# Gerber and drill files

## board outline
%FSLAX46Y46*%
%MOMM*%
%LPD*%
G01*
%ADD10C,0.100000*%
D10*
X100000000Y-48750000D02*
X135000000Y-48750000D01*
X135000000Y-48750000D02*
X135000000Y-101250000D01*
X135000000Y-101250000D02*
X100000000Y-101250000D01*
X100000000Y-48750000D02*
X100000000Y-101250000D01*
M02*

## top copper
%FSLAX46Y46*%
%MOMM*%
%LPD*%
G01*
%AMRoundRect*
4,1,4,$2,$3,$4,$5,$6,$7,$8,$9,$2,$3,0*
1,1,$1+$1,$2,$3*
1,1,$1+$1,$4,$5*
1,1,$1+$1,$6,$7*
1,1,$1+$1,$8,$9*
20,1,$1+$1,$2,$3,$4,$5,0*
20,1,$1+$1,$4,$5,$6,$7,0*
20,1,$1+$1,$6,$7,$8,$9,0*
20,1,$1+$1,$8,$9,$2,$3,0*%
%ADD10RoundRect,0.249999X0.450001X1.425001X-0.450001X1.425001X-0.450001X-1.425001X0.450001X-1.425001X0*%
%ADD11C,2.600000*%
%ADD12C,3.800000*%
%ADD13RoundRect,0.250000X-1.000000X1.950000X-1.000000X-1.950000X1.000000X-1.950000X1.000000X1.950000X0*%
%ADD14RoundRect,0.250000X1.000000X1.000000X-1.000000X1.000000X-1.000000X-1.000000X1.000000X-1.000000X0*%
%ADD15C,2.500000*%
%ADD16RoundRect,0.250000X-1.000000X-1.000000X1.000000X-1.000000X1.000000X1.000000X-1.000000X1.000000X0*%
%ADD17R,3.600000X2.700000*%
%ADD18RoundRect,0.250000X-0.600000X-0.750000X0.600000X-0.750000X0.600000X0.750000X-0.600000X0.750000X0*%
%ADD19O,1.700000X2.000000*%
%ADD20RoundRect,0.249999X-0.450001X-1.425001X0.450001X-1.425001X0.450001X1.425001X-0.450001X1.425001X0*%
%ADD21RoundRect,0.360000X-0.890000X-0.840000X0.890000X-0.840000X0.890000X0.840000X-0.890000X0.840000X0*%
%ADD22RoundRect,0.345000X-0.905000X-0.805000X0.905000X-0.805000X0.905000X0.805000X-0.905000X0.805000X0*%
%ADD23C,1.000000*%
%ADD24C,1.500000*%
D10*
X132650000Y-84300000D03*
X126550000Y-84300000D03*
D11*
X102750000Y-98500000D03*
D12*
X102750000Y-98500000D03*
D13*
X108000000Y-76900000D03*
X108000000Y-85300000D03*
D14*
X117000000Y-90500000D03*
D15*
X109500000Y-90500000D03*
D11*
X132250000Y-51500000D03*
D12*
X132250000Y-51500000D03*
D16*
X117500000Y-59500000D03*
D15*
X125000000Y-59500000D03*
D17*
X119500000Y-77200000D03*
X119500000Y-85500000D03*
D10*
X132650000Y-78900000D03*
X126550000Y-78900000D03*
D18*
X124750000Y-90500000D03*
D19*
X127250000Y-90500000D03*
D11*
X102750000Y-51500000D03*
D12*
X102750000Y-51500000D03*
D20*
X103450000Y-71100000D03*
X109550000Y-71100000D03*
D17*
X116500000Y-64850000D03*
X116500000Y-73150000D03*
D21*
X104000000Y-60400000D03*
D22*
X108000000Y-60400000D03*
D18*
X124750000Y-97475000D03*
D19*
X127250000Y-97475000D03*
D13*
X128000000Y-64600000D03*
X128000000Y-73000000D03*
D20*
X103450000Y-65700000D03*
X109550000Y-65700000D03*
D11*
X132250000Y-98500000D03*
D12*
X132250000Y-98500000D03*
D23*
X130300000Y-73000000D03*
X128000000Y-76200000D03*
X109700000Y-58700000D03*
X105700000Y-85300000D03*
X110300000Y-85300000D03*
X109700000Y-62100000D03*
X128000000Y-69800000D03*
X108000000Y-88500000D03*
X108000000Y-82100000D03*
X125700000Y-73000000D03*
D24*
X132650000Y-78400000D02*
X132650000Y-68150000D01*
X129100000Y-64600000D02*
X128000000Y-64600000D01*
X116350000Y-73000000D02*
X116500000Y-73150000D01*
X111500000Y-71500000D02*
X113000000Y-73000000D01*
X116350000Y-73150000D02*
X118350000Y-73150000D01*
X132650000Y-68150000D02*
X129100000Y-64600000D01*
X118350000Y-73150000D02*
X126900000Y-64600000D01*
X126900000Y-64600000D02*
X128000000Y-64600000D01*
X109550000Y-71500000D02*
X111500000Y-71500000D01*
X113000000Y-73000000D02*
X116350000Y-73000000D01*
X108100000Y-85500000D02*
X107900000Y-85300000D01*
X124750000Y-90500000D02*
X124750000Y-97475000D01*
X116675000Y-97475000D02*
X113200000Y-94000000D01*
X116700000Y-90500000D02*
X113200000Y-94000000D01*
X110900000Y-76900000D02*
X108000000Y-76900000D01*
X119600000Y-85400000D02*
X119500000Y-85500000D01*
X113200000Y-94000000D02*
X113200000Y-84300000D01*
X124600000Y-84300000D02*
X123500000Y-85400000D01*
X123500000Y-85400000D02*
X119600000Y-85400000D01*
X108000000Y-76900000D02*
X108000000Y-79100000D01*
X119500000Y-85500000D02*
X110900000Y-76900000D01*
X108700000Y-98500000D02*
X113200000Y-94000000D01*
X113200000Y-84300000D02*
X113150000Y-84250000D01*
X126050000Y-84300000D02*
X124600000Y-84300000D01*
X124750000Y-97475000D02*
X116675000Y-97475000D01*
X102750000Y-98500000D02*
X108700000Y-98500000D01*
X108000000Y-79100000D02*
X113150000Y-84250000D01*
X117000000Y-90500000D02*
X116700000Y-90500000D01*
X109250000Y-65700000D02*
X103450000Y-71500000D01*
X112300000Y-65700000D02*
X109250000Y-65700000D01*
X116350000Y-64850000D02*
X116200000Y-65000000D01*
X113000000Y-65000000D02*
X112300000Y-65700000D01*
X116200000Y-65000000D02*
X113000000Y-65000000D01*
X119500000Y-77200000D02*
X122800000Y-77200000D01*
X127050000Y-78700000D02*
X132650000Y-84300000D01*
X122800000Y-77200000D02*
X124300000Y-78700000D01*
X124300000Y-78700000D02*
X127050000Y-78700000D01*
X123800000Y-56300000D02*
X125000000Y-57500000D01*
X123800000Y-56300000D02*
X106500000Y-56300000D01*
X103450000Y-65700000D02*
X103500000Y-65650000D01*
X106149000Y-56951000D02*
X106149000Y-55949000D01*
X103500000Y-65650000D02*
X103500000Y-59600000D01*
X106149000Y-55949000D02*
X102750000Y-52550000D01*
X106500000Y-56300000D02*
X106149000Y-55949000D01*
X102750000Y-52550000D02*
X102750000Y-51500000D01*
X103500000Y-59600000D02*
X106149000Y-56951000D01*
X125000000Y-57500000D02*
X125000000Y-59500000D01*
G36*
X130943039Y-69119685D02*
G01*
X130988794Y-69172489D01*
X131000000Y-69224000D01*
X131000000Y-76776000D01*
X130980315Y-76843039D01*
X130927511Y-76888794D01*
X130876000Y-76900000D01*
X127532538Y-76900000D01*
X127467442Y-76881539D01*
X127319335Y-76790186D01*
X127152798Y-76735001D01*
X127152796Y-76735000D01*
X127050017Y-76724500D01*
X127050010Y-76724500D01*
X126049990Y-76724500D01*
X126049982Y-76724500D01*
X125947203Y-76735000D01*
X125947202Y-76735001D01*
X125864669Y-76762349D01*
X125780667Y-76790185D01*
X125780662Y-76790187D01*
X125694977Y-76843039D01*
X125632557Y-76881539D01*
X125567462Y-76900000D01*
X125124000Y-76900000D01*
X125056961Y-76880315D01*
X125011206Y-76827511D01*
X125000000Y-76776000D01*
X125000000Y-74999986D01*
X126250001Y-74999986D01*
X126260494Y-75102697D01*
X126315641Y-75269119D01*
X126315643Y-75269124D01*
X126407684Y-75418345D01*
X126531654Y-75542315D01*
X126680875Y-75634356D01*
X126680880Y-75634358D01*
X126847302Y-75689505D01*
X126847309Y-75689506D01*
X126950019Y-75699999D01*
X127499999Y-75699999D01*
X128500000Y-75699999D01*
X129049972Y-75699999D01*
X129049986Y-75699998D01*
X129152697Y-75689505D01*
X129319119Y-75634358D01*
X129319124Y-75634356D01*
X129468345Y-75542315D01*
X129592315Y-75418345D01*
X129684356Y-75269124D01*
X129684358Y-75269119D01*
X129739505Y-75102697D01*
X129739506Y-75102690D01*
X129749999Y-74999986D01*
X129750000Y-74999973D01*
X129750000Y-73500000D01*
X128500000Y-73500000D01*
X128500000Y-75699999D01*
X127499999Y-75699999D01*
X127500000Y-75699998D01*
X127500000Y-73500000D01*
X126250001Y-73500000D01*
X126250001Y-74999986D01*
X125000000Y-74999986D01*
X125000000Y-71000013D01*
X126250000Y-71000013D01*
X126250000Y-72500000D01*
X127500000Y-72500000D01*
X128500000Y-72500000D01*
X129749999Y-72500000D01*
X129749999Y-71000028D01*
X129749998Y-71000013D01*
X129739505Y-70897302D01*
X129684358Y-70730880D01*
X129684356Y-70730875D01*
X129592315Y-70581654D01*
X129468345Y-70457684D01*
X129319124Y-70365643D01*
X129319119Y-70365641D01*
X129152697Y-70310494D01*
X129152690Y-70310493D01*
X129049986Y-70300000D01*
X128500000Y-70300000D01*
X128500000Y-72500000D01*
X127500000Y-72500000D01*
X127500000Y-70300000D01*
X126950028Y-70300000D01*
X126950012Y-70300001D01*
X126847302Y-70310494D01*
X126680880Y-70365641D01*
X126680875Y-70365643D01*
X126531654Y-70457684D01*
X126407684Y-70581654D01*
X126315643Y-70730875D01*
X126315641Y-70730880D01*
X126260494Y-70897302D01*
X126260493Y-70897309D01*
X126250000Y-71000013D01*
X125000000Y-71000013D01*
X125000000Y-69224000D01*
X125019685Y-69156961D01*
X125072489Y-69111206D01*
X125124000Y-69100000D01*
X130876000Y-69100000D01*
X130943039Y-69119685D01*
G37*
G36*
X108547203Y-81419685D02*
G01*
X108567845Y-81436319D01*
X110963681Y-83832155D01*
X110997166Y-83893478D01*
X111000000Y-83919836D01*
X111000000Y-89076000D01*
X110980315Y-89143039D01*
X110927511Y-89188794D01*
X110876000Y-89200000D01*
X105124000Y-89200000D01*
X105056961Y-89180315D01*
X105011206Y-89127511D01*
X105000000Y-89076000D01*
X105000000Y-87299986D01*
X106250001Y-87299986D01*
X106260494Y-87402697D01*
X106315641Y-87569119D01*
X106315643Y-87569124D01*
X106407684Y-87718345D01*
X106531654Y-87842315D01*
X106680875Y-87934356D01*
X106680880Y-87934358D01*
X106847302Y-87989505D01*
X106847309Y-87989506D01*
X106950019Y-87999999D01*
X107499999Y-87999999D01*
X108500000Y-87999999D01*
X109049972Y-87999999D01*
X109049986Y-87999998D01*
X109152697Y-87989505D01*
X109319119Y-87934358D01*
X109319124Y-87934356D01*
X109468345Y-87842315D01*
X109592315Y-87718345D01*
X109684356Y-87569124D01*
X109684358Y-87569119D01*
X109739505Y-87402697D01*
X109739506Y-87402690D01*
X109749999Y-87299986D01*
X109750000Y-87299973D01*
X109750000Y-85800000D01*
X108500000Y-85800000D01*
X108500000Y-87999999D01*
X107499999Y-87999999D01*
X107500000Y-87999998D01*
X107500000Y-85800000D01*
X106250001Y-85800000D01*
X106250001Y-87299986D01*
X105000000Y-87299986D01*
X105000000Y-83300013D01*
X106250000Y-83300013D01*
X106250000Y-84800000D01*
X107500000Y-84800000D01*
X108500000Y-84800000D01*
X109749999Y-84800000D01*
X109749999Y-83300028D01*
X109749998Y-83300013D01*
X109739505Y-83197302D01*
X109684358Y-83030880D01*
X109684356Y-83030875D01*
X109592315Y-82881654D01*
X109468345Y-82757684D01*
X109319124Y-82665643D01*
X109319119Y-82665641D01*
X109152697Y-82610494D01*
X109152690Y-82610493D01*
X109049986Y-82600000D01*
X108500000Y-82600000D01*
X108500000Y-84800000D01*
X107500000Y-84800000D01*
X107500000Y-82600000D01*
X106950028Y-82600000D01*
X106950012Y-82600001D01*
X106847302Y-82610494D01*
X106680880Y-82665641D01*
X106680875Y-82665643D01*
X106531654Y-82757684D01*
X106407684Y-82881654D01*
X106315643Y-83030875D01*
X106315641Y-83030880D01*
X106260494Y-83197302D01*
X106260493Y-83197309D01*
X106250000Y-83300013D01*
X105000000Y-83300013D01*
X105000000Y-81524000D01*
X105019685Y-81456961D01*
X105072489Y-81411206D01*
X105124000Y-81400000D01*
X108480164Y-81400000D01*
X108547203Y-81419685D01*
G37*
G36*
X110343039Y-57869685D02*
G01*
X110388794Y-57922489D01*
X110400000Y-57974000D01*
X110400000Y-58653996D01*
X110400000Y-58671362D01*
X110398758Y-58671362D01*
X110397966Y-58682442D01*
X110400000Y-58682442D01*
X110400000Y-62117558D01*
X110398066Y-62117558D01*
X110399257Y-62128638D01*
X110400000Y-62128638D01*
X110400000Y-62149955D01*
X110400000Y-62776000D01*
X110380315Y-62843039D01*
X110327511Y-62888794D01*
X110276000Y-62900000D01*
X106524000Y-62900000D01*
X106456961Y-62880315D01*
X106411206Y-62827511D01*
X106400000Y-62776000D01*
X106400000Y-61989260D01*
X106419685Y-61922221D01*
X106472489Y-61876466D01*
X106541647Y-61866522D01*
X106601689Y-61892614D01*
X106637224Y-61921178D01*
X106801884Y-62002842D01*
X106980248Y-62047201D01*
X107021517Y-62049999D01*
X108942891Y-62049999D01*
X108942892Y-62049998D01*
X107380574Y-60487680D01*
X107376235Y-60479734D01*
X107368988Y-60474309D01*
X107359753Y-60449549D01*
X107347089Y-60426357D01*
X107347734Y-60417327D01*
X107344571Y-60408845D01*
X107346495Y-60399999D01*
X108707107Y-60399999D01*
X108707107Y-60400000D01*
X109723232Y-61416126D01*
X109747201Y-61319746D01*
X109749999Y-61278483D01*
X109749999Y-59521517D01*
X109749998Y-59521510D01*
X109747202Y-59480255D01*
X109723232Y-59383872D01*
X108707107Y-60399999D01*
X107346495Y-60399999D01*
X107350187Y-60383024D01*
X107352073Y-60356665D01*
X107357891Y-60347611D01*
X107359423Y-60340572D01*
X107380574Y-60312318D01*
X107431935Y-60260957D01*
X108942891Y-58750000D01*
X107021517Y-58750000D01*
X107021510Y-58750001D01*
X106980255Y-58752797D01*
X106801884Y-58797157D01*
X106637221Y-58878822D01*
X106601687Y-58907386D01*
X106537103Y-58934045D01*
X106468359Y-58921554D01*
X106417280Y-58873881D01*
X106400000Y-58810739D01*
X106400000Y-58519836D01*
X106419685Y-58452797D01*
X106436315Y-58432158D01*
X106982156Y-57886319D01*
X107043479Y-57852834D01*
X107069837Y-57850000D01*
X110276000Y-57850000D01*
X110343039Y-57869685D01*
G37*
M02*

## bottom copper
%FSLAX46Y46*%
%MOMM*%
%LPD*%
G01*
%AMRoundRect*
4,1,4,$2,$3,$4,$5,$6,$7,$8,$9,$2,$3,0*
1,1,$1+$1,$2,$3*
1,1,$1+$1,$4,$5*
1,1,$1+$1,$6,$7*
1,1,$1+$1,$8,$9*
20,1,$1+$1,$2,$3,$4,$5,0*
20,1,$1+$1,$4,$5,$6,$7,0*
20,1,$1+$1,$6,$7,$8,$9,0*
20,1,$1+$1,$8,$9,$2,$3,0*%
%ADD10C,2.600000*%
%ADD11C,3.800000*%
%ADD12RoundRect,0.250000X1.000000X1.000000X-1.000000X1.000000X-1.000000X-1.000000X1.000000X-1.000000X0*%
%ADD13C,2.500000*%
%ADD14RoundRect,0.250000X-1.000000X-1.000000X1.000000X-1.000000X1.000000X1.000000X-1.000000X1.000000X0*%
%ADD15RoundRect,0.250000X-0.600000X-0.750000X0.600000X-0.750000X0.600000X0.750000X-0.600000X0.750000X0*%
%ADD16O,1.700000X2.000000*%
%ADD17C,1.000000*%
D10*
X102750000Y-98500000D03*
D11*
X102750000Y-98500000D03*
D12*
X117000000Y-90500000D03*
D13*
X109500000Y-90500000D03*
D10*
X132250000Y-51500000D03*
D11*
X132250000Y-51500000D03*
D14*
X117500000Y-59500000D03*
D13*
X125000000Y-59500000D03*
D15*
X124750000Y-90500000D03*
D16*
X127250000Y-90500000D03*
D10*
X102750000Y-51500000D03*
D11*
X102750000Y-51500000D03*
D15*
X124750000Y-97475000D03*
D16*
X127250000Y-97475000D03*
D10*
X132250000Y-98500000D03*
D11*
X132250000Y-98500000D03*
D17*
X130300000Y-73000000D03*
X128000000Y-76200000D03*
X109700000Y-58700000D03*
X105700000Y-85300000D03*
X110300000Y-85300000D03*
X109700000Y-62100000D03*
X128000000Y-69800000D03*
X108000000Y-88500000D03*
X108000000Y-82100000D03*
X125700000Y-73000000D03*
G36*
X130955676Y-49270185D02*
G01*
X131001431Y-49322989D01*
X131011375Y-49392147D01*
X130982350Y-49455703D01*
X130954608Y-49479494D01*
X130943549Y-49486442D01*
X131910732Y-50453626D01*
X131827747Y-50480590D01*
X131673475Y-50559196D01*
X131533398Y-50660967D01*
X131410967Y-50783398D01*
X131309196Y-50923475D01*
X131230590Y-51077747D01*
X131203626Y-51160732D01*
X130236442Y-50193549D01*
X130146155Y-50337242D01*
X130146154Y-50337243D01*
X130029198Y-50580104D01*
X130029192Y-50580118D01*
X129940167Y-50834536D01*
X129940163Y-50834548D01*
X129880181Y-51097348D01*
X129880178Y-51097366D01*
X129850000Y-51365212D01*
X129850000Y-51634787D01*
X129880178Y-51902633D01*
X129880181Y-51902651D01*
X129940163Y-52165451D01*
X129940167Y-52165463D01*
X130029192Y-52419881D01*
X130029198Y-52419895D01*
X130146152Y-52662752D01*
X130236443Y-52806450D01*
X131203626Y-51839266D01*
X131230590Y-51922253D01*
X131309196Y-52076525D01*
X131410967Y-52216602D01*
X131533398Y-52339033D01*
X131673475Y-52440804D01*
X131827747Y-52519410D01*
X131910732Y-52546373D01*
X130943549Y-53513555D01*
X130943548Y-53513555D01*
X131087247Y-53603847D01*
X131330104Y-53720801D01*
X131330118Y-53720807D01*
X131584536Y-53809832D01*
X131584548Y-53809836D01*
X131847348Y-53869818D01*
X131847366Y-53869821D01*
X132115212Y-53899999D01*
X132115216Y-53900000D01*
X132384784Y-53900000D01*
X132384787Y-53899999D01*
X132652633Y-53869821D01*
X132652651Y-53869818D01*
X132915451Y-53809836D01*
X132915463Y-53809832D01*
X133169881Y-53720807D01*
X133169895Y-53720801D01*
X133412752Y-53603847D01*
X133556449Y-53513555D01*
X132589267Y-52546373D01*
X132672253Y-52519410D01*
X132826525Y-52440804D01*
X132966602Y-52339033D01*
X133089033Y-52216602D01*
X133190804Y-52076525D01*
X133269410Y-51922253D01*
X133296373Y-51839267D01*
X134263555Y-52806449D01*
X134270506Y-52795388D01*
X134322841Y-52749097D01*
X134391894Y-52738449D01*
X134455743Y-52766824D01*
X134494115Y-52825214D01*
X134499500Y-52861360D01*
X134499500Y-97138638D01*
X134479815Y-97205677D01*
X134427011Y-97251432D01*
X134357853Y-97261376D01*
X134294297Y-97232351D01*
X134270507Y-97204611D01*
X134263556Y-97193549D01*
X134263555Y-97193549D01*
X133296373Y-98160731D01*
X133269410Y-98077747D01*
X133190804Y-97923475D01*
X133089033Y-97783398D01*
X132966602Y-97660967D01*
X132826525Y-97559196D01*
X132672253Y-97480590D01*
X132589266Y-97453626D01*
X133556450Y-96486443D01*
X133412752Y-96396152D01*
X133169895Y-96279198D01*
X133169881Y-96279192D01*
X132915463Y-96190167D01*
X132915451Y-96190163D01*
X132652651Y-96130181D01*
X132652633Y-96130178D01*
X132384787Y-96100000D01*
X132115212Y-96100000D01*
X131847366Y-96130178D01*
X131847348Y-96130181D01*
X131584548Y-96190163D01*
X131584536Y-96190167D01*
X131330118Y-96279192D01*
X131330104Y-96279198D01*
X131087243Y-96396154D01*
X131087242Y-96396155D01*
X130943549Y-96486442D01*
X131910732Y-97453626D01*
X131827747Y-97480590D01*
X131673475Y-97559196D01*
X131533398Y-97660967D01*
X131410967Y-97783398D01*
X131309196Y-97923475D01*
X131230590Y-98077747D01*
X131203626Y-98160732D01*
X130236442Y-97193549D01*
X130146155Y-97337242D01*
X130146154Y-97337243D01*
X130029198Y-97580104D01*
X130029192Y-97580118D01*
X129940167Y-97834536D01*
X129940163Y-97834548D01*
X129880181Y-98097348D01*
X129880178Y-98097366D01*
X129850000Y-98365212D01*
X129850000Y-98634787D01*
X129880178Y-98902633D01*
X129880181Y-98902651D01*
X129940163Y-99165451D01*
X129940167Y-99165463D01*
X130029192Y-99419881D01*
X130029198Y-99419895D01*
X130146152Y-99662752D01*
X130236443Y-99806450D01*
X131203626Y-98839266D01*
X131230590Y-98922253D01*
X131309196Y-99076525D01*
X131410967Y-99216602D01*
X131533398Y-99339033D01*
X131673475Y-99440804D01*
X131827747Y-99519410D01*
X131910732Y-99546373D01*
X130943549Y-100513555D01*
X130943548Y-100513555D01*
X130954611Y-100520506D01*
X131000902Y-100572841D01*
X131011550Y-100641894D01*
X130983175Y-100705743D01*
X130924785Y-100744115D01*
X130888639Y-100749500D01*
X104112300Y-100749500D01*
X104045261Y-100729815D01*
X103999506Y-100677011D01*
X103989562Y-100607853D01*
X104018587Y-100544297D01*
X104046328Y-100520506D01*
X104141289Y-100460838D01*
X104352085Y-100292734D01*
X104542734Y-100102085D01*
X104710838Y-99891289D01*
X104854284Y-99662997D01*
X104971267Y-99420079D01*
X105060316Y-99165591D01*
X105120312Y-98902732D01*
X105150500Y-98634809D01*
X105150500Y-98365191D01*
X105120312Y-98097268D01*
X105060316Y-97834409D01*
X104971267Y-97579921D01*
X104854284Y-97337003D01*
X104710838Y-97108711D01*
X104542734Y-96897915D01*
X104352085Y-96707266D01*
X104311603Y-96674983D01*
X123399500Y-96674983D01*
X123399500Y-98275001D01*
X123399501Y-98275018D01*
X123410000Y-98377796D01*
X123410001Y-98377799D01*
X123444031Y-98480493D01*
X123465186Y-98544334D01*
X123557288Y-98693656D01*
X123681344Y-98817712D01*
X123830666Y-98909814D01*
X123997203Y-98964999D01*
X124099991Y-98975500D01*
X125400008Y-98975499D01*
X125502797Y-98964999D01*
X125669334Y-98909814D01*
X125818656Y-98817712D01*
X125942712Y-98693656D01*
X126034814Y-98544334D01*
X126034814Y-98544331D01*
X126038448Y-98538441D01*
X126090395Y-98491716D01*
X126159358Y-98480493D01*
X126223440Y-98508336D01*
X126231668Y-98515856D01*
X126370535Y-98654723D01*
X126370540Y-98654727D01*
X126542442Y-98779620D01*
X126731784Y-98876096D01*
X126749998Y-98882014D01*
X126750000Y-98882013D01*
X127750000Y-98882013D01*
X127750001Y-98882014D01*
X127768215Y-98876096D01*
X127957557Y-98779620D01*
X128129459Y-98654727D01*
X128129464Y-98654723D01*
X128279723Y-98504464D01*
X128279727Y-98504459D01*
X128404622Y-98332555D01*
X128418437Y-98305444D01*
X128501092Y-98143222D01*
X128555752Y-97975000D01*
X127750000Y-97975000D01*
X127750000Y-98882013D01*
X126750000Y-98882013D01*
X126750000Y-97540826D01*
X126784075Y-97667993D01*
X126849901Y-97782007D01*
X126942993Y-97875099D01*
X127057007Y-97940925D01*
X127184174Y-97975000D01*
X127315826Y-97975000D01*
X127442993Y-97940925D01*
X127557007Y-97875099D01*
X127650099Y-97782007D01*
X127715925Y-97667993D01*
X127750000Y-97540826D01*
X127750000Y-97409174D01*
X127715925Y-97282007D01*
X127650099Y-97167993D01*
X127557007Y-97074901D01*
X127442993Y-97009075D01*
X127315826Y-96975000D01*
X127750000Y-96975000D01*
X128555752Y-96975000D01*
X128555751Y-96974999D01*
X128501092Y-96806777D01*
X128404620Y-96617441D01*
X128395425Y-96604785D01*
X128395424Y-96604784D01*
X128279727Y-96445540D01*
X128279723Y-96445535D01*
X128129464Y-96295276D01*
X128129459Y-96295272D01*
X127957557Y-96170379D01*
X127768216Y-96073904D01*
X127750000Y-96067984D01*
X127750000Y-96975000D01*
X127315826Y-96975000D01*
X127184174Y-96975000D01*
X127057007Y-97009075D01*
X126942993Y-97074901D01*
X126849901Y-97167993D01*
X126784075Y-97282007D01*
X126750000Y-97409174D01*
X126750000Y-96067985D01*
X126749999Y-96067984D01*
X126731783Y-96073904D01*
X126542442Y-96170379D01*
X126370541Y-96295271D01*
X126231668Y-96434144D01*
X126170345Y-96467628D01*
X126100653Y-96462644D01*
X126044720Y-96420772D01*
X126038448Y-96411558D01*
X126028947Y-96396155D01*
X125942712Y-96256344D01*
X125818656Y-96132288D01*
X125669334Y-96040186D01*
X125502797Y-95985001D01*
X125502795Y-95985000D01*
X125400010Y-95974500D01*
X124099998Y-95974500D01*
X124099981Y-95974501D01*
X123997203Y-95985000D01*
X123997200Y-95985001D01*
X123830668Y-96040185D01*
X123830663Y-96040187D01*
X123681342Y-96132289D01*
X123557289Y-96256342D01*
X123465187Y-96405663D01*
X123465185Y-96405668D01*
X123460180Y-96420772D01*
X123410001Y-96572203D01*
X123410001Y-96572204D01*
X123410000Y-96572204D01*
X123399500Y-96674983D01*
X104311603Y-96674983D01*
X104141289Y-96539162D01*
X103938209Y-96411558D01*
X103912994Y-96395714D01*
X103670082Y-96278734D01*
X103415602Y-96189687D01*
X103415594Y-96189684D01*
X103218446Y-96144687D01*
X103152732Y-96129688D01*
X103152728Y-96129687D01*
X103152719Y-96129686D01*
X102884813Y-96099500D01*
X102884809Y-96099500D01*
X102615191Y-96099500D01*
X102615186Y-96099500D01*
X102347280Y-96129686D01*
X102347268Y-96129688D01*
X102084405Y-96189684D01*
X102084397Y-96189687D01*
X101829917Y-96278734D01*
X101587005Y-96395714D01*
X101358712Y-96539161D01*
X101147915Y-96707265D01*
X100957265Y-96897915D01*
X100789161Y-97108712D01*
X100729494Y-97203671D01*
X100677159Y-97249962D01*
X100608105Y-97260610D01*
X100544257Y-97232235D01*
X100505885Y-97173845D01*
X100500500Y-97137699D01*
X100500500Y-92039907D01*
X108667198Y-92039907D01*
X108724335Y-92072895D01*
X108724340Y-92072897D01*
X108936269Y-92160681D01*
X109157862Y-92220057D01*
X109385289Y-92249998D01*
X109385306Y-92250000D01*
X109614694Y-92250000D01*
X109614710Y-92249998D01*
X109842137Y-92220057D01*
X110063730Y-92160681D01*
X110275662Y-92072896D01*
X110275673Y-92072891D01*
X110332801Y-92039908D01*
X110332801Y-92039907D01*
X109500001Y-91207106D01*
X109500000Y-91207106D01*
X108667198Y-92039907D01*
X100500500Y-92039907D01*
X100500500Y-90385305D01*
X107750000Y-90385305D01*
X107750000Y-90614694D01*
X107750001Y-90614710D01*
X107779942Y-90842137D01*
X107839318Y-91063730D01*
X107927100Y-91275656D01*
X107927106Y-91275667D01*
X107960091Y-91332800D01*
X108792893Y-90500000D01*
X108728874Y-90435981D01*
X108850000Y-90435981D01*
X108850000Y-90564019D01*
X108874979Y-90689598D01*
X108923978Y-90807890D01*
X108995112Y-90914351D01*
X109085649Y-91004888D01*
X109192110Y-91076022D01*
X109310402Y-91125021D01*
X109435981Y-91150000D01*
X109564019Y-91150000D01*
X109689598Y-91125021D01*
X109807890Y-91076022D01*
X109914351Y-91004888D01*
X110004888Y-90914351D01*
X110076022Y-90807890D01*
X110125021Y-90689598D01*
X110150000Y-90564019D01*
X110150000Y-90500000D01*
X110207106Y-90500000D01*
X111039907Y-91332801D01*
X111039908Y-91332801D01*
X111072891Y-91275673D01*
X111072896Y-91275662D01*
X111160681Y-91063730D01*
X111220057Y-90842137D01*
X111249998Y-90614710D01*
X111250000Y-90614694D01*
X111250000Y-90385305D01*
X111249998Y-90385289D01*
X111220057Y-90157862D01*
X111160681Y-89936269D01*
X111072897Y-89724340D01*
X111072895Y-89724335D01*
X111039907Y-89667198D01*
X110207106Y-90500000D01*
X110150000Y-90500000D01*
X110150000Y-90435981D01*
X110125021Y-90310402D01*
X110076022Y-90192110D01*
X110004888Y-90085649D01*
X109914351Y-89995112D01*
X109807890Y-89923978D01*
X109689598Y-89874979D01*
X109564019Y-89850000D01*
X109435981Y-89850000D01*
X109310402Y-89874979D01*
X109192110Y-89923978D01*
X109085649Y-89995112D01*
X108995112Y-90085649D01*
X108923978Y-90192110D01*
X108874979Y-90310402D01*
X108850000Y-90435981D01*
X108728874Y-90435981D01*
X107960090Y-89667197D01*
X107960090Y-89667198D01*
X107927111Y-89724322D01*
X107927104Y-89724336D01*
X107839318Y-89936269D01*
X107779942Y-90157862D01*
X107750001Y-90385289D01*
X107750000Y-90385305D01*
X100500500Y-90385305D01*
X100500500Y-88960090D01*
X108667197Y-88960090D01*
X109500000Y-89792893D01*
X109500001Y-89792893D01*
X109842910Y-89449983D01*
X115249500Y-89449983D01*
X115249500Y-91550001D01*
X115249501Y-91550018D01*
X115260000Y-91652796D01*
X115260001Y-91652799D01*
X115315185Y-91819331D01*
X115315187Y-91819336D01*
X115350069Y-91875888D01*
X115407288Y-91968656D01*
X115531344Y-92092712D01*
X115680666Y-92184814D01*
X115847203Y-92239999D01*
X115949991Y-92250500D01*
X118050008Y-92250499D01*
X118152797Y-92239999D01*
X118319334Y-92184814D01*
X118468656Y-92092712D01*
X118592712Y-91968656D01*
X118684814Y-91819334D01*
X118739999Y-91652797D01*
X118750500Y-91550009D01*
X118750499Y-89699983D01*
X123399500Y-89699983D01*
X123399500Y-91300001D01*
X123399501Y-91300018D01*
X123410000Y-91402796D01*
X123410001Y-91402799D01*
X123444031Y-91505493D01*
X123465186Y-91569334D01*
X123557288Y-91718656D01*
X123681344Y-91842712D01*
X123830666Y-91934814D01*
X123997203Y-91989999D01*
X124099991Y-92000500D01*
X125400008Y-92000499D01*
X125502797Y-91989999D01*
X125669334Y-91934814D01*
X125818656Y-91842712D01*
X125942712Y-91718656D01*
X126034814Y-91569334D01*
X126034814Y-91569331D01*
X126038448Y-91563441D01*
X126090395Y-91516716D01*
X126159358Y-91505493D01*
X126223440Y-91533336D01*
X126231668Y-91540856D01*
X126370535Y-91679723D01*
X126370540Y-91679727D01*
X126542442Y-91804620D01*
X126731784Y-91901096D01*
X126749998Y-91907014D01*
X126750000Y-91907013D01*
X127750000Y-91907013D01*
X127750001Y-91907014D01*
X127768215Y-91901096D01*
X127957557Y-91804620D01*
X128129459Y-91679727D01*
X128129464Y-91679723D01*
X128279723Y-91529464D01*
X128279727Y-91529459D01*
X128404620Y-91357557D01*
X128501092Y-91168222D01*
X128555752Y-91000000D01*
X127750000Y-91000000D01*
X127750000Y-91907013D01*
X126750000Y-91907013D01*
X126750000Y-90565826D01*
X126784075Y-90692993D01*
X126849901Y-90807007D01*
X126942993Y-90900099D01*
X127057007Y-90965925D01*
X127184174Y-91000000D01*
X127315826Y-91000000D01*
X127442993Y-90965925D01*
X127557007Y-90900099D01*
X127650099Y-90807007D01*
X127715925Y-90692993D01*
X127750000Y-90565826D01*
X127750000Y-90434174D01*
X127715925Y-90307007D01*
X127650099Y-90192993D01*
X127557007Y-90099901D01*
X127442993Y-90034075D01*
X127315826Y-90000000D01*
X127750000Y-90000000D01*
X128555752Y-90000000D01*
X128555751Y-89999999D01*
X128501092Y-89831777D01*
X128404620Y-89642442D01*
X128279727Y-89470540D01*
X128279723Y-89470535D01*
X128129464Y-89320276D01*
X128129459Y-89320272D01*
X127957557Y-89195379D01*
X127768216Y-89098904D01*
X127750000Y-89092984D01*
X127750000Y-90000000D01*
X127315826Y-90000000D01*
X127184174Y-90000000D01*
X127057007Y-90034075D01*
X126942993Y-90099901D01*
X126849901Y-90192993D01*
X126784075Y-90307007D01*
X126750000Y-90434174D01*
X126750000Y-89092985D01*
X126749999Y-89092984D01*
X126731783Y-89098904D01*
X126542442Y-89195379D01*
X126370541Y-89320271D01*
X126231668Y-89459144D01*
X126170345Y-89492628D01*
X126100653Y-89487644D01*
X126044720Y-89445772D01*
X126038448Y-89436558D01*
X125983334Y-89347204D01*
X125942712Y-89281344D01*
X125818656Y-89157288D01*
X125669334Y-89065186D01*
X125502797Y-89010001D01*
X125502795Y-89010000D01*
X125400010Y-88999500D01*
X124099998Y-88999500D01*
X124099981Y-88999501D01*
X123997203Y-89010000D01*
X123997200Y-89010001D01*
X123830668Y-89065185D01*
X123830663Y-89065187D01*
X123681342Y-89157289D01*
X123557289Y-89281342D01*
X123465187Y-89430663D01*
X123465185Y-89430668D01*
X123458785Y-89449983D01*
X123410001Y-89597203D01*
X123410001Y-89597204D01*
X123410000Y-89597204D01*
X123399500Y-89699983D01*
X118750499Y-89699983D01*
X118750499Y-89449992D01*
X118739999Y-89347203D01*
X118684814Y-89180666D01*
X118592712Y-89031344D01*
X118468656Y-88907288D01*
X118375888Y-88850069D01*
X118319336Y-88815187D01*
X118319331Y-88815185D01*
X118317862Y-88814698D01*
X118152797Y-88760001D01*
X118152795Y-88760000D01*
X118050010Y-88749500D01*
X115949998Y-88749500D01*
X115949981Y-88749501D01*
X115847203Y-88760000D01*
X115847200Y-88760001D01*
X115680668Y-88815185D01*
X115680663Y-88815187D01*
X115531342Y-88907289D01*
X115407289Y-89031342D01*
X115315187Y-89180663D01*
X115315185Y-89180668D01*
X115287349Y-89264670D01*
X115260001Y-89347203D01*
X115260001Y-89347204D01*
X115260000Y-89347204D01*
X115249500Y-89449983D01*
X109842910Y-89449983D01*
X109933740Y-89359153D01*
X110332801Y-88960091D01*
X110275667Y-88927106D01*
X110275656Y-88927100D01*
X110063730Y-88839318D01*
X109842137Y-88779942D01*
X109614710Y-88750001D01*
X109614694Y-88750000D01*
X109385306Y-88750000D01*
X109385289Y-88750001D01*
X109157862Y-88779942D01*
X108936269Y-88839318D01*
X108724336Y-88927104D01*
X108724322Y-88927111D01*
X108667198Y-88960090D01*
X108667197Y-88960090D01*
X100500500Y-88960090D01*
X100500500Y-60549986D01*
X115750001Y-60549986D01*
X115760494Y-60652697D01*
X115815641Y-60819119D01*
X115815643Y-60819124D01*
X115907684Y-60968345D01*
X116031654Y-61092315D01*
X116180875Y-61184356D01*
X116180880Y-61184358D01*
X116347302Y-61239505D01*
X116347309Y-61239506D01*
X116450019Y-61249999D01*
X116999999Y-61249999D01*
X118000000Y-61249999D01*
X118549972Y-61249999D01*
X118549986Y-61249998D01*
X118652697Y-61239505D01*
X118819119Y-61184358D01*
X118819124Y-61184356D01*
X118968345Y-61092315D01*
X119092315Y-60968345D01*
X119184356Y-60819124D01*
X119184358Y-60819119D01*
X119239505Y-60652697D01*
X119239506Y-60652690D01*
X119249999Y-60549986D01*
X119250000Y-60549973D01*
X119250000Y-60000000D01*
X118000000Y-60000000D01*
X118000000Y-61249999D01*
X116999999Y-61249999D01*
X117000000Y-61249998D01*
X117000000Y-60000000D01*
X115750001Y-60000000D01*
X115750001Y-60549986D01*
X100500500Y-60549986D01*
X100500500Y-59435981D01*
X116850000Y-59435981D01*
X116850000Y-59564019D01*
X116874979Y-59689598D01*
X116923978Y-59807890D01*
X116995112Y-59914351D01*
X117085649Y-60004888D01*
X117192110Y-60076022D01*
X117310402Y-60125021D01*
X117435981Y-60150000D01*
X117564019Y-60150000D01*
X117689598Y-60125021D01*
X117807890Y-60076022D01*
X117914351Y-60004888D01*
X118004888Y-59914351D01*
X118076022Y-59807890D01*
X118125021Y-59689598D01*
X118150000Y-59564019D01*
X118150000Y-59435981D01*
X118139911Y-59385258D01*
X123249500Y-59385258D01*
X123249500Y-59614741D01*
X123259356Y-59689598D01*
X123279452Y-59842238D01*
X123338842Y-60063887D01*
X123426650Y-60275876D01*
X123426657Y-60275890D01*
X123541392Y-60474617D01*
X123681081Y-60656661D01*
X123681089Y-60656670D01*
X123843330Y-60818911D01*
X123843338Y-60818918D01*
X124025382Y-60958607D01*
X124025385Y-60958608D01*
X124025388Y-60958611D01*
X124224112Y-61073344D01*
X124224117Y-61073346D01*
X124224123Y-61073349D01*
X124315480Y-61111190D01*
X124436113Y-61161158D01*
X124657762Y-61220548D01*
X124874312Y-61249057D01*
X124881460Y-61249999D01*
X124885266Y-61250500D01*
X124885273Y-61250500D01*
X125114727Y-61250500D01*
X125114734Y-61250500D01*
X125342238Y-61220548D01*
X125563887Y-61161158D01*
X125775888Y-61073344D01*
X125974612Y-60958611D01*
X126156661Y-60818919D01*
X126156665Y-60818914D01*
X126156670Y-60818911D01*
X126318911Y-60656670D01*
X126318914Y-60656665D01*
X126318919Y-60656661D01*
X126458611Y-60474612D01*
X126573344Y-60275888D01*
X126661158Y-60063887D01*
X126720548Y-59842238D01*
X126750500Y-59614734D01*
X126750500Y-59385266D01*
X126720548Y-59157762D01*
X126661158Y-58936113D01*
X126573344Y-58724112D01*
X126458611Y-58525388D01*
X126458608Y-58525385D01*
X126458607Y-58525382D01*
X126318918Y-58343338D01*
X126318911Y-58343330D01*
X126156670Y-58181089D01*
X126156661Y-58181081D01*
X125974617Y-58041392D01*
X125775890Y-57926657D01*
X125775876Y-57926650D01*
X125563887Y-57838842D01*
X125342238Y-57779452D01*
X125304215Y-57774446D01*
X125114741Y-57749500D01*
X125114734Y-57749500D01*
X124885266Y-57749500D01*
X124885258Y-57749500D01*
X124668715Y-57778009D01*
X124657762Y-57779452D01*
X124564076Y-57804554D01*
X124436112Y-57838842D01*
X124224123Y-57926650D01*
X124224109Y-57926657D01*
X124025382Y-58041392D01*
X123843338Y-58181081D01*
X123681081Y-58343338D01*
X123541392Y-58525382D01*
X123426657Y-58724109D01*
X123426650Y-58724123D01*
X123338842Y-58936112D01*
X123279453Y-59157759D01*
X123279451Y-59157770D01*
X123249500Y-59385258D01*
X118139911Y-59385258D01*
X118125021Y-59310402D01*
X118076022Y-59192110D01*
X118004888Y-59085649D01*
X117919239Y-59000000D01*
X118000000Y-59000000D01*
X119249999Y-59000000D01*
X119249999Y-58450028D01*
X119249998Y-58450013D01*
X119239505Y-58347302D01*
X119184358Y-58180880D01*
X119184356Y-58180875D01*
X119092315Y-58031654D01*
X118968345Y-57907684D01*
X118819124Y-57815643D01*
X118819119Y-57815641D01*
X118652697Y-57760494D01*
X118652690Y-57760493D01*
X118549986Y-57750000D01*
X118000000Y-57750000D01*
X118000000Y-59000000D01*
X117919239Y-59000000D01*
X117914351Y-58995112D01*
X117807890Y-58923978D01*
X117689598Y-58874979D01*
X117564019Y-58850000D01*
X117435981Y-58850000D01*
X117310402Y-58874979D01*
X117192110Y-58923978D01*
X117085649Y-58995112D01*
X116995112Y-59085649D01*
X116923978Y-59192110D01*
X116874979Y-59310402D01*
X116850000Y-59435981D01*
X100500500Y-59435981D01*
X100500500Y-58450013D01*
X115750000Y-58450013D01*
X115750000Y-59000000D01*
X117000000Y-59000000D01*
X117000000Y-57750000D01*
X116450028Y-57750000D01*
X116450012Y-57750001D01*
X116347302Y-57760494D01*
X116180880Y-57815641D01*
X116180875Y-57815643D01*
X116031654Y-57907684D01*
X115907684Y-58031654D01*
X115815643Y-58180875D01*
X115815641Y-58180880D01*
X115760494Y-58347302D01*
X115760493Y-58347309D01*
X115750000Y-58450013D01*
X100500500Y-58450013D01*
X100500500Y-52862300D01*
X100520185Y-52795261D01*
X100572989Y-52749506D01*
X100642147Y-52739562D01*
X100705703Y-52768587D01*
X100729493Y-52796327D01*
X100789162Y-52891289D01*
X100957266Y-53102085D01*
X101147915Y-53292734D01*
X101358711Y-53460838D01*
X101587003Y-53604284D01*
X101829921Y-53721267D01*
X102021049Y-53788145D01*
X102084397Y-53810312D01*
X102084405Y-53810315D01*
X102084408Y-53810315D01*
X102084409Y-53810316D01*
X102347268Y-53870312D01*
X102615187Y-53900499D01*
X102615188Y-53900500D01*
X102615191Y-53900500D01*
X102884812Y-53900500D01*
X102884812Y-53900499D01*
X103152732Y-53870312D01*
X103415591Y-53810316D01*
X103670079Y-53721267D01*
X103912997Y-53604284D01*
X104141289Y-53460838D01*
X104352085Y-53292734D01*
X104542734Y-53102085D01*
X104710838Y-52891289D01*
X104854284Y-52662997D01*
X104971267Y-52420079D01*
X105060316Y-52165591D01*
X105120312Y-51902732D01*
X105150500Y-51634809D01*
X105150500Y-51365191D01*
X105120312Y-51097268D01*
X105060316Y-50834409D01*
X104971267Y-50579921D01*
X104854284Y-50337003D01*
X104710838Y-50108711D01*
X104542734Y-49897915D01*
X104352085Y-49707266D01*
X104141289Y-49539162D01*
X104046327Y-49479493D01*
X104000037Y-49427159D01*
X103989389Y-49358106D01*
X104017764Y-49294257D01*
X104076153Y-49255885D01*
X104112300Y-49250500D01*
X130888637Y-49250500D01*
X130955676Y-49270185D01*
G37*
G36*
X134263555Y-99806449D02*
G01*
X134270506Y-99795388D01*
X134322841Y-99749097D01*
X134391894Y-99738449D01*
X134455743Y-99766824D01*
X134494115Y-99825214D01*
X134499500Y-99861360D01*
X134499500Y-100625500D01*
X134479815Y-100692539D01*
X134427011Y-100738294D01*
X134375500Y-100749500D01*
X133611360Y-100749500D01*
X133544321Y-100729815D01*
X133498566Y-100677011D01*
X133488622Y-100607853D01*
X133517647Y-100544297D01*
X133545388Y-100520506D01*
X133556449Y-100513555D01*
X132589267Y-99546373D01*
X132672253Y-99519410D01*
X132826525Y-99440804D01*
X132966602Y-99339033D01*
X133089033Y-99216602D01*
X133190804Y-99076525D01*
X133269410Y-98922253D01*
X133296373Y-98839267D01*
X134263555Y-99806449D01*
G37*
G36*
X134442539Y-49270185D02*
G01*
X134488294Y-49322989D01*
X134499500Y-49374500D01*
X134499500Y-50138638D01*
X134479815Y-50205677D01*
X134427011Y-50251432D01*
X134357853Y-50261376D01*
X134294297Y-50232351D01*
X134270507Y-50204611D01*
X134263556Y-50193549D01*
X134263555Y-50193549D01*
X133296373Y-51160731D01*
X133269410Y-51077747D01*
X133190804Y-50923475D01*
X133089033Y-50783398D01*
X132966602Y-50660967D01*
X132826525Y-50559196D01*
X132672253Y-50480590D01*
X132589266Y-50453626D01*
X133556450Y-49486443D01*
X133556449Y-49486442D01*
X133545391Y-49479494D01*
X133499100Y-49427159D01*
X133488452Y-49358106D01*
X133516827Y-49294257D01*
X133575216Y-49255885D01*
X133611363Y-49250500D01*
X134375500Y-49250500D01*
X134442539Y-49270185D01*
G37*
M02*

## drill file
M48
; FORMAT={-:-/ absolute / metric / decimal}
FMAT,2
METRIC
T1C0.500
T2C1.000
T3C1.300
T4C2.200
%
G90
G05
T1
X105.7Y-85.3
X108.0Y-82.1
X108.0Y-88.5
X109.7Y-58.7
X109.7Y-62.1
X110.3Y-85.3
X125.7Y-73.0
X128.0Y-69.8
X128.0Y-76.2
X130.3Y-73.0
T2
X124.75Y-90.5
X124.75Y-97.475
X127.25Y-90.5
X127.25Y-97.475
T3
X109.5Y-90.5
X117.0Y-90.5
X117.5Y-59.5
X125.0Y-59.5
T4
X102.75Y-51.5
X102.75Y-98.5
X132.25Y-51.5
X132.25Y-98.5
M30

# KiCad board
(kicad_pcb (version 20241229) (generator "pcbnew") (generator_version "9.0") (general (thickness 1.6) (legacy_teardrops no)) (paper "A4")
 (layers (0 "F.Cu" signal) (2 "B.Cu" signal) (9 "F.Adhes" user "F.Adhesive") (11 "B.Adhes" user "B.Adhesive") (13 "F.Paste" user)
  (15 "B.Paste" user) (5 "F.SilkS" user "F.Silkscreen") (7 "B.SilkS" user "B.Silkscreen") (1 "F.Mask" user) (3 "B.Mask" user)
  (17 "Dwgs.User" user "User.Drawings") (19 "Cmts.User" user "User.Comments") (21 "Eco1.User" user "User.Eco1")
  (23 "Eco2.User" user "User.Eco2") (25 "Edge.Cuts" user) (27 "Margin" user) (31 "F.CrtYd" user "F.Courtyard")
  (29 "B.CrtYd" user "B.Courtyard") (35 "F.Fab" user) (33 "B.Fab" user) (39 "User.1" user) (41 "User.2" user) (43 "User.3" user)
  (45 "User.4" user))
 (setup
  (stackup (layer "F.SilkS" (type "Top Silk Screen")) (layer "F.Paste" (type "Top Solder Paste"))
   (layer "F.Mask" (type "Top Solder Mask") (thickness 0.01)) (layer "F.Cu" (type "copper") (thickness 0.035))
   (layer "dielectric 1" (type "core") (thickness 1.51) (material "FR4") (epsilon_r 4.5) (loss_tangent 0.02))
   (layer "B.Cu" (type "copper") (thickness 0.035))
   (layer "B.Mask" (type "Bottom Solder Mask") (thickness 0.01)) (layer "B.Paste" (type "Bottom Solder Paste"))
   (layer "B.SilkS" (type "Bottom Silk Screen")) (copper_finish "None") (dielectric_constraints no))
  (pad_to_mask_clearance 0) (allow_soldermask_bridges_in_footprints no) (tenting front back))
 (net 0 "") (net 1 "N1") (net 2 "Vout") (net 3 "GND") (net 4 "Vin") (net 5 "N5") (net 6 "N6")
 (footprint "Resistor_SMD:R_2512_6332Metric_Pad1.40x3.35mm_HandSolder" (layer "F.Cu") (at 129.6 84.3 180)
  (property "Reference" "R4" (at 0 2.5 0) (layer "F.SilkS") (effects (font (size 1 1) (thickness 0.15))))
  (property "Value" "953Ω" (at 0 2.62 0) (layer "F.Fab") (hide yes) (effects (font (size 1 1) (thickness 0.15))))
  (pad "1" smd roundrect (at -3.05 0 180) (size 1.4 3.35) (layers "F.Cu" "F.Mask" "F.Paste") (roundrect_rratio 0.178571) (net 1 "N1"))
  (pad "2" smd roundrect (at 3.05 0 180) (size 1.4 3.35) (layers "F.Cu" "F.Mask" "F.Paste") (roundrect_rratio 0.178571) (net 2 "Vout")))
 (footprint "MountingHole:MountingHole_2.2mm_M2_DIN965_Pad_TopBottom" (layer "F.Cu") (at 102.75 98.5)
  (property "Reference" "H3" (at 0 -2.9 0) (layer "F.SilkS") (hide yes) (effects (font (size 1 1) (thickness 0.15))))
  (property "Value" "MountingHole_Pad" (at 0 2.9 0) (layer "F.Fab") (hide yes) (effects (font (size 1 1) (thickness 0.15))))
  (pad "1" thru_hole circle (at 0 0) (size 2.6 2.6) (drill 2.2) (layers "*.Cu" "*.Mask") (remove_unused_layers no) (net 2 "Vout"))
  (pad "1" connect circle (at 0 0) (size 3.8 3.8) (layers "F.Cu" "F.Mask") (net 2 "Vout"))
  (pad "1" connect circle (at 0 0) (size 3.8 3.8) (layers "B.Cu" "B.Mask") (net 2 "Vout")))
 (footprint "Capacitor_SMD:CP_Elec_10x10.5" (layer "F.Cu") (at 108 81.1 -90)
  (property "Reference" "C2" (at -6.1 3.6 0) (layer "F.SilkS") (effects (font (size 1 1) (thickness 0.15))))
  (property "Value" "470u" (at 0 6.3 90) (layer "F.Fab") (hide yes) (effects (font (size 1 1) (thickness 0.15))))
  (pad "1" smd roundrect (at -4.2 0 270) (size 4.4 2.5) (layers "F.Cu" "F.Mask" "F.Paste") (roundrect_rratio 0.1) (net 2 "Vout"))
  (pad "2" smd roundrect (at 4.2 0 270) (size 4.4 2.5) (layers "F.Cu" "F.Mask" "F.Paste") (roundrect_rratio 0.1) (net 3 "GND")))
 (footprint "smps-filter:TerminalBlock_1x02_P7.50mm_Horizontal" (layer "F.Cu") (at 117 90.5 180)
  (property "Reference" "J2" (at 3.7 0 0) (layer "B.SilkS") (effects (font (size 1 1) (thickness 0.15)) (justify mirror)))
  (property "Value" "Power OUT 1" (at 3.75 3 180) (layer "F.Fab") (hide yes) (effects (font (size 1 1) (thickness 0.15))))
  (pad "1" thru_hole roundrect (at 0 0 180) (size 2.5 2.5) (drill 1.3) (layers "*.Cu" "*.Mask") (remove_unused_layers no)
   (roundrect_rratio 0.1) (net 2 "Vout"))
  (pad "2" thru_hole circle (at 7.5 0 180) (size 2.5 2.5) (drill 1.3) (layers "*.Cu" "*.Mask") (remove_unused_layers no) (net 3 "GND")))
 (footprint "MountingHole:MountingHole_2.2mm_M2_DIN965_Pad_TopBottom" (layer "F.Cu") (at 132.25 51.5)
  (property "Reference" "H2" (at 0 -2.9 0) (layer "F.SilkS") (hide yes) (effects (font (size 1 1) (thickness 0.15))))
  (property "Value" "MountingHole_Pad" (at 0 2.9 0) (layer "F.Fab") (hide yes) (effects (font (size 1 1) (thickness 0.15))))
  (pad "1" thru_hole circle (at 0 0) (size 2.6 2.6) (drill 2.2) (layers "*.Cu" "*.Mask") (remove_unused_layers no) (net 3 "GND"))
  (pad "1" connect circle (at 0 0) (size 3.8 3.8) (layers "F.Cu" "F.Mask") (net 3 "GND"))
  (pad "1" connect circle (at 0 0) (size 3.8 3.8) (layers "B.Cu" "B.Mask") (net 3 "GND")))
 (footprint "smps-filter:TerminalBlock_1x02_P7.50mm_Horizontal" (layer "F.Cu") (at 117.5 59.5)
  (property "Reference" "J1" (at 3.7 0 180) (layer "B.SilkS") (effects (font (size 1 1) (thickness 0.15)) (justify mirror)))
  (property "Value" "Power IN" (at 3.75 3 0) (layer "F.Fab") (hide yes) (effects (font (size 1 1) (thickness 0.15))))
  (pad "1" thru_hole roundrect (at 0 0) (size 2.5 2.5) (drill 1.3) (layers "*.Cu" "*.Mask") (remove_unused_layers no) (roundrect_rratio 0.1)
   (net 3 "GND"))
  (pad "2" thru_hole circle (at 7.5 0) (size 2.5 2.5) (drill 1.3) (layers "*.Cu" "*.Mask") (remove_unused_layers no) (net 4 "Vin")))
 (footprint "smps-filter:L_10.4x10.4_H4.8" (layer "F.Cu") (at 119.5 81.35 -90)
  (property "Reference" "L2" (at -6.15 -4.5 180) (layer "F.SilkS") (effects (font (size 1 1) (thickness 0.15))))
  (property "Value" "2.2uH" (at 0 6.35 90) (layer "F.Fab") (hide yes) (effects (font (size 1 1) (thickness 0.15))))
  (pad "1" smd rect (at -4.15 0 270) (size 2.7 3.6) (layers "F.Cu" "F.Mask" "F.Paste") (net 1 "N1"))
  (pad "2" smd rect (at 4.15 0 270) (size 2.7 3.6) (layers "F.Cu" "F.Mask" "F.Paste") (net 2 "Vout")))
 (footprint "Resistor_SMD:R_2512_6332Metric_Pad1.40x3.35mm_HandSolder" (layer "F.Cu") (at 129.6 78.9 180)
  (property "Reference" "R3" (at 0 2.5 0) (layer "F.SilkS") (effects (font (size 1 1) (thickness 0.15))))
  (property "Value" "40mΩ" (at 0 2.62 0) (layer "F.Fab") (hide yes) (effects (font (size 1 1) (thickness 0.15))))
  (pad "1" smd roundrect (at -3.05 0 180) (size 1.4 3.35) (layers "F.Cu" "F.Mask" "F.Paste") (roundrect_rratio 0.178571) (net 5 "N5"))
  (pad "2" smd roundrect (at 3.05 0 180) (size 1.4 3.35) (layers "F.Cu" "F.Mask" "F.Paste") (roundrect_rratio 0.178571) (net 1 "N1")))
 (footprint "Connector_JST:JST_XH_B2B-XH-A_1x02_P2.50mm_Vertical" (layer "F.Cu") (at 124.75 90.5)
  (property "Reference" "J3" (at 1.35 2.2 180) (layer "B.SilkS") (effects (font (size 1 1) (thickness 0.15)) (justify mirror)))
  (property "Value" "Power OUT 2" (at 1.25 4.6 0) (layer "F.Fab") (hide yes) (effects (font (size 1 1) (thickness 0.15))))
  (pad "1" thru_hole roundrect (at 0 0) (size 1.7 2) (drill 1) (layers "*.Cu" "*.Mask") (remove_unused_layers no)
   (roundrect_rratio 0.147059) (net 2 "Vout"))
  (pad "2" thru_hole oval (at 2.5 0) (size 1.7 2) (drill 1) (layers "*.Cu" "*.Mask") (remove_unused_layers no) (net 3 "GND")))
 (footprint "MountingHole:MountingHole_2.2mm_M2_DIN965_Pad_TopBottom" (layer "F.Cu") (at 102.75 51.5)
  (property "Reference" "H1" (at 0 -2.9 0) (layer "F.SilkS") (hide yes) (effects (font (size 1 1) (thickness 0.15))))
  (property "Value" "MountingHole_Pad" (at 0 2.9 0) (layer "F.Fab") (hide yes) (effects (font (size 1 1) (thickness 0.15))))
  (pad "1" thru_hole circle (at 0 0) (size 2.6 2.6) (drill 2.2) (layers "*.Cu" "*.Mask") (remove_unused_layers no) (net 4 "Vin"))
  (pad "1" connect circle (at 0 0) (size 3.8 3.8) (layers "F.Cu" "F.Mask") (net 4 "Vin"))
  (pad "1" connect circle (at 0 0) (size 3.8 3.8) (layers "B.Cu" "B.Mask") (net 4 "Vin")))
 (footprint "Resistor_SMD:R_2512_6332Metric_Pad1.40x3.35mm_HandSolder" (layer "F.Cu") (at 106.5 71.1)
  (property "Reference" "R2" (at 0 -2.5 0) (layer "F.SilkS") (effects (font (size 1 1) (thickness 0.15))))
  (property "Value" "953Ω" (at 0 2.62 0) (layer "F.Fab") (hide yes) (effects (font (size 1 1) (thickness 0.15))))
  (pad "1" smd roundrect (at -3.05 0) (size 1.4 3.35) (layers "F.Cu" "F.Mask" "F.Paste") (roundrect_rratio 0.178571) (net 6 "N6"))
  (pad "2" smd roundrect (at 3.05 0) (size 1.4 3.35) (layers "F.Cu" "F.Mask" "F.Paste") (roundrect_rratio 0.178571) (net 5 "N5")))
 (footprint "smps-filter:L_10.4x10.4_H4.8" (layer "F.Cu") (at 116.5 69 -90)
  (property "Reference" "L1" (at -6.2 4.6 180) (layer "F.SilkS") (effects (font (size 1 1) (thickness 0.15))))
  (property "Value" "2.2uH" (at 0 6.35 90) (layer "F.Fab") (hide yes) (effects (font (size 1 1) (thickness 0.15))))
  (pad "1" smd rect (at -4.15 0 270) (size 2.7 3.6) (layers "F.Cu" "F.Mask" "F.Paste") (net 6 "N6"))
  (pad "2" smd rect (at 4.15 0 270) (size 2.7 3.6) (layers "F.Cu" "F.Mask" "F.Paste") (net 5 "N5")))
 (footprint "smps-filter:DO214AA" (layer "F.Cu") (at 106 60.4)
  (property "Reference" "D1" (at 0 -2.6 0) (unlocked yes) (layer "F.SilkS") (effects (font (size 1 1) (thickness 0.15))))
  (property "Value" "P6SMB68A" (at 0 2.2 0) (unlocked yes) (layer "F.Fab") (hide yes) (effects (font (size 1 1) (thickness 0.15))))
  (pad "1" smd roundrect (at -2 0) (size 2.5 2.4) (layers "F.Cu" "F.Mask" "F.Paste") (roundrect_rratio 0.15) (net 4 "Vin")
   (thermal_bridge_angle 45)
   (padstack (mode front_inner_back)
    (layer "Inner" (shape roundrect) (size 2.2 2.3) (roundrect_rratio 0.15) (thermal_bridge_angle 45) (zone_connect -1))
    (layer "B.Cu" (shape roundrect) (size 2.2 2.3) (roundrect_rratio 0.15) (thermal_bridge_angle 45) (zone_connect -1))))
  (pad "2" smd roundrect (at 2 0) (size 2.5 2.3) (layers "F.Cu" "F.Mask" "F.Paste") (roundrect_rratio 0.15) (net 3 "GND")
   (thermal_bridge_angle 45)
   (padstack (mode front_inner_back)
    (layer "Inner" (shape roundrect) (size 2.2 2.3) (roundrect_rratio 0.15) (thermal_bridge_angle 45) (zone_connect -1))
    (layer "B.Cu" (shape roundrect) (size 2.2 2.3) (roundrect_rratio 0.15) (thermal_bridge_angle 45) (zone_connect -1)))))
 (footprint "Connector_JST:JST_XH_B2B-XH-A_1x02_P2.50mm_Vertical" (layer "F.Cu") (at 124.75 97.475)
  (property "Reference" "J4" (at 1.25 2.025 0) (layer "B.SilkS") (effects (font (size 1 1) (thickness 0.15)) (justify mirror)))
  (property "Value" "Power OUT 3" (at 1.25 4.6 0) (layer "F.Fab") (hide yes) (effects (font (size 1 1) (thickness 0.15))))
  (pad "1" thru_hole roundrect (at 0 0) (size 1.7 2) (drill 1) (layers "*.Cu" "*.Mask") (remove_unused_layers no)
   (roundrect_rratio 0.147059) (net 2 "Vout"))
  (pad "2" thru_hole oval (at 2.5 0) (size 1.7 2) (drill 1) (layers "*.Cu" "*.Mask") (remove_unused_layers no) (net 3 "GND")))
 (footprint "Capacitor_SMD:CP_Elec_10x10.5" (layer "F.Cu") (at 128 68.8 -90)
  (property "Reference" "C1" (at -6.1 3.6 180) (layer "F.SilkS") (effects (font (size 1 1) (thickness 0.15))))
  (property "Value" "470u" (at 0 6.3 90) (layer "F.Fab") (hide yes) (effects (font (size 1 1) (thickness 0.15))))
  (pad "1" smd roundrect (at -4.2 0 270) (size 4.4 2.5) (layers "F.Cu" "F.Mask" "F.Paste") (roundrect_rratio 0.1) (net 5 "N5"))
  (pad "2" smd roundrect (at 4.2 0 270) (size 4.4 2.5) (layers "F.Cu" "F.Mask" "F.Paste") (roundrect_rratio 0.1) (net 3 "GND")))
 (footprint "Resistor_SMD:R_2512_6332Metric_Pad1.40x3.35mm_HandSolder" (layer "F.Cu") (at 106.5 65.7)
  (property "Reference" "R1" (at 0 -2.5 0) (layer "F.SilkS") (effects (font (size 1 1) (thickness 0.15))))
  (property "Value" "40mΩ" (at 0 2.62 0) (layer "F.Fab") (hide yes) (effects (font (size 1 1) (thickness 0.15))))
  (pad "1" smd roundrect (at -3.05 0) (size 1.4 3.35) (layers "F.Cu" "F.Mask" "F.Paste") (roundrect_rratio 0.178571) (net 4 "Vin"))
  (pad "2" smd roundrect (at 3.05 0) (size 1.4 3.35) (layers "F.Cu" "F.Mask" "F.Paste") (roundrect_rratio 0.178571) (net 6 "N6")))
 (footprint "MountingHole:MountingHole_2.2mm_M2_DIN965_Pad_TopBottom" (layer "B.Cu") (at 132.25 98.5)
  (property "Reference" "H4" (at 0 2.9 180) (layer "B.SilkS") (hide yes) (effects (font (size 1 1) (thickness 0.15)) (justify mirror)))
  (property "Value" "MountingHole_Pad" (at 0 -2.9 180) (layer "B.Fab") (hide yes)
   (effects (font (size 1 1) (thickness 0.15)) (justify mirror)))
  (pad "1" thru_hole circle (at 0 0) (size 2.6 2.6) (drill 2.2) (layers "*.Cu" "*.Mask") (remove_unused_layers no) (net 3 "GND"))
  (pad "1" connect circle (at 0 0) (size 3.8 3.8) (layers "F.Cu" "F.Mask") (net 3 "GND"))
  (pad "1" connect circle (at 0 0) (size 3.8 3.8) (layers "B.Cu" "B.Mask") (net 3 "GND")))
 (gr_line (start 100 48.75) (end 135 48.75) (stroke (width 0.1) (type solid)) (layer "Edge.Cuts"))
 (gr_line (start 135 48.75) (end 135 101.25) (stroke (width 0.1) (type solid)) (layer "Edge.Cuts"))
 (gr_line (start 135 101.25) (end 100 101.25) (stroke (width 0.1) (type solid)) (layer "Edge.Cuts"))
 (gr_line (start 100 48.75) (end 100 101.25) (stroke (width 0.1) (type solid)) (layer "Edge.Cuts"))
 (segment (start 132.65 78.4) (end 132.65 68.15) (width 1.5) (layer "F.Cu") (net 5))
 (segment (start 129.1 64.6) (end 128 64.6) (width 1.5) (layer "F.Cu") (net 5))
 (segment (start 116.35 73) (end 116.5 73.15) (width 1.5) (layer "F.Cu") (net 5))
 (segment (start 111.5 71.5) (end 113 73) (width 1.5) (layer "F.Cu") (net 5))
 (segment (start 116.35 73.15) (end 118.35 73.15) (width 1.5) (layer "F.Cu") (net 5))
 (segment (start 132.65 68.15) (end 129.1 64.6) (width 1.5) (layer "F.Cu") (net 5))
 (segment (start 118.35 73.15) (end 126.9 64.6) (width 1.5) (layer "F.Cu") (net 5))
 (segment (start 126.9 64.6) (end 128 64.6) (width 1.5) (layer "F.Cu") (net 5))
 (segment (start 109.55 71.5) (end 111.5 71.5) (width 1.5) (layer "F.Cu") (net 5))
 (segment (start 113 73) (end 116.35 73) (width 1.5) (layer "F.Cu") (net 5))
 (segment (start 108.1 85.5) (end 107.9 85.3) (width 1.5) (layer "F.Cu") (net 3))
 (via (at 130.3 73) (size 1) (drill 0.5) (layers "F.Cu" "B.Cu") (free yes) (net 3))
 (via (at 128 76.2) (size 1) (drill 0.5) (layers "F.Cu" "B.Cu") (free yes) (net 3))
 (via (at 109.7 58.7) (size 1) (drill 0.5) (layers "F.Cu" "B.Cu") (free yes) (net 3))
 (via (at 105.7 85.3) (size 1) (drill 0.5) (layers "F.Cu" "B.Cu") (free yes) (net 3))
 (via (at 110.3 85.3) (size 1) (drill 0.5) (layers "F.Cu" "B.Cu") (free yes) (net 3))
 (via (at 109.7 62.1) (size 1) (drill 0.5) (layers "F.Cu" "B.Cu") (free yes) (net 3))
 (via (at 128 69.8) (size 1) (drill 0.5) (layers "F.Cu" "B.Cu") (free yes) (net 3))
 (via (at 108 88.5) (size 1) (drill 0.5) (layers "F.Cu" "B.Cu") (free yes) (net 3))
 (via (at 108 82.1) (size 1) (drill 0.5) (layers "F.Cu" "B.Cu") (free yes) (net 3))
 (via (at 125.7 73) (size 1) (drill 0.5) (layers "F.Cu" "B.Cu") (free yes) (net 3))
 (segment (start 124.75 90.5) (end 124.75 97.475) (width 1.5) (layer "F.Cu") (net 2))
 (segment (start 116.675 97.475) (end 113.2 94) (width 1.5) (layer "F.Cu") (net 2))
 (segment (start 116.7 90.5) (end 113.2 94) (width 1.5) (layer "F.Cu") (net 2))
 (segment (start 110.9 76.9) (end 108 76.9) (width 1.5) (layer "F.Cu") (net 2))
 (segment (start 119.6 85.4) (end 119.5 85.5) (width 1.5) (layer "F.Cu") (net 2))
 (segment (start 113.2 94) (end 113.2 84.3) (width 1.5) (layer "F.Cu") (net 2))
 (segment (start 124.6 84.3) (end 123.5 85.4) (width 1.5) (layer "F.Cu") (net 2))
 (segment (start 123.5 85.4) (end 119.6 85.4) (width 1.5) (layer "F.Cu") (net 2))
 (segment (start 108 76.9) (end 108 79.1) (width 1.5) (layer "F.Cu") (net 2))
 (segment (start 119.5 85.5) (end 110.9 76.9) (width 1.5) (layer "F.Cu") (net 2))
 (segment (start 108.7 98.5) (end 113.2 94) (width 1.5) (layer "F.Cu") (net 2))
 (segment (start 113.2 84.3) (end 113.15 84.25) (width 1.5) (layer "F.Cu") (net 2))
 (segment (start 126.05 84.3) (end 124.6 84.3) (width 1.5) (layer "F.Cu") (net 2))
 (segment (start 124.75 97.475) (end 116.675 97.475) (width 1.5) (layer "F.Cu") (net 2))
 (segment (start 102.75 98.5) (end 108.7 98.5) (width 1.5) (layer "F.Cu") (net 2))
 (segment (start 108 79.1) (end 113.15 84.25) (width 1.5) (layer "F.Cu") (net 2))
 (segment (start 117 90.5) (end 116.7 90.5) (width 1.5) (layer "F.Cu") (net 2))
 (segment (start 109.25 65.7) (end 103.45 71.5) (width 1.5) (layer "F.Cu") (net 6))
 (segment (start 112.3 65.7) (end 109.25 65.7) (width 1.5) (layer "F.Cu") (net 6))
 (segment (start 116.35 64.85) (end 116.2 65) (width 1.5) (layer "F.Cu") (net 6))
 (segment (start 113 65) (end 112.3 65.7) (width 1.5) (layer "F.Cu") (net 6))
 (segment (start 116.2 65) (end 113 65) (width 1.5) (layer "F.Cu") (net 6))
 (segment (start 119.5 77.2) (end 122.8 77.2) (width 1.5) (layer "F.Cu") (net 1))
 (segment (start 127.05 78.7) (end 132.65 84.3) (width 1.5) (layer "F.Cu") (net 1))
 (segment (start 122.8 77.2) (end 124.3 78.7) (width 1.5) (layer "F.Cu") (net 1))
 (segment (start 124.3 78.7) (end 127.05 78.7) (width 1.5) (layer "F.Cu") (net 1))
 (segment (start 123.8 56.3) (end 125 57.5) (width 1.5) (layer "F.Cu") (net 4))
 (segment (start 123.8 56.3) (end 106.5 56.3) (width 1.5) (layer "F.Cu") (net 4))
 (segment (start 103.45 65.7) (end 103.5 65.65) (width 1.5) (layer "F.Cu") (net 4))
 (segment (start 106.149 56.951) (end 106.149 55.949) (width 1.5) (layer "F.Cu") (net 4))
 (segment (start 103.5 65.65) (end 103.5 59.6) (width 1.5) (layer "F.Cu") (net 4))
 (segment (start 106.149 55.949) (end 102.75 52.55) (width 1.5) (layer "F.Cu") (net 4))
 (segment (start 106.5 56.3) (end 106.149 55.949) (width 1.5) (layer "F.Cu") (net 4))
 (segment (start 102.75 52.55) (end 102.75 51.5) (width 1.5) (layer "F.Cu") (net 4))
 (segment (start 103.5 59.6) (end 106.149 56.951) (width 1.5) (layer "F.Cu") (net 4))
 (segment (start 125 57.5) (end 125 59.5) (width 1.5) (layer "F.Cu") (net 4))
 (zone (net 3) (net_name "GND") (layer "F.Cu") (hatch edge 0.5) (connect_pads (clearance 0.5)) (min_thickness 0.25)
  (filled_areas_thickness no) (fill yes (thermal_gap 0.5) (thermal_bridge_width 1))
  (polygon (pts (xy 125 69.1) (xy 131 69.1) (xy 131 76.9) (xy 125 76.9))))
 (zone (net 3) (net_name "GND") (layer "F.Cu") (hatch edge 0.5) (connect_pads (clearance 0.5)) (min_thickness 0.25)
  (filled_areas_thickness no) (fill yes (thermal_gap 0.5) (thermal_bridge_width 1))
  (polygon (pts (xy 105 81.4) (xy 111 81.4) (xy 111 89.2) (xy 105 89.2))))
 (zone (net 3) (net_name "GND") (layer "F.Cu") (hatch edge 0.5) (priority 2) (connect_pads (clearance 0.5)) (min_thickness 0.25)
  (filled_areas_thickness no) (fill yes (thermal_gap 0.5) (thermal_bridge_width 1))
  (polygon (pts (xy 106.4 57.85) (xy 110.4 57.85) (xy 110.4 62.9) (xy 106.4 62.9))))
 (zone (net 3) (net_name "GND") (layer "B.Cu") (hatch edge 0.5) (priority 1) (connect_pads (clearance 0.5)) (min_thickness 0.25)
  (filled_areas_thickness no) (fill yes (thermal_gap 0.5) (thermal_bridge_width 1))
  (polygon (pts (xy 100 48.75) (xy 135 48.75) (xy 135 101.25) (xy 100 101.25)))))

